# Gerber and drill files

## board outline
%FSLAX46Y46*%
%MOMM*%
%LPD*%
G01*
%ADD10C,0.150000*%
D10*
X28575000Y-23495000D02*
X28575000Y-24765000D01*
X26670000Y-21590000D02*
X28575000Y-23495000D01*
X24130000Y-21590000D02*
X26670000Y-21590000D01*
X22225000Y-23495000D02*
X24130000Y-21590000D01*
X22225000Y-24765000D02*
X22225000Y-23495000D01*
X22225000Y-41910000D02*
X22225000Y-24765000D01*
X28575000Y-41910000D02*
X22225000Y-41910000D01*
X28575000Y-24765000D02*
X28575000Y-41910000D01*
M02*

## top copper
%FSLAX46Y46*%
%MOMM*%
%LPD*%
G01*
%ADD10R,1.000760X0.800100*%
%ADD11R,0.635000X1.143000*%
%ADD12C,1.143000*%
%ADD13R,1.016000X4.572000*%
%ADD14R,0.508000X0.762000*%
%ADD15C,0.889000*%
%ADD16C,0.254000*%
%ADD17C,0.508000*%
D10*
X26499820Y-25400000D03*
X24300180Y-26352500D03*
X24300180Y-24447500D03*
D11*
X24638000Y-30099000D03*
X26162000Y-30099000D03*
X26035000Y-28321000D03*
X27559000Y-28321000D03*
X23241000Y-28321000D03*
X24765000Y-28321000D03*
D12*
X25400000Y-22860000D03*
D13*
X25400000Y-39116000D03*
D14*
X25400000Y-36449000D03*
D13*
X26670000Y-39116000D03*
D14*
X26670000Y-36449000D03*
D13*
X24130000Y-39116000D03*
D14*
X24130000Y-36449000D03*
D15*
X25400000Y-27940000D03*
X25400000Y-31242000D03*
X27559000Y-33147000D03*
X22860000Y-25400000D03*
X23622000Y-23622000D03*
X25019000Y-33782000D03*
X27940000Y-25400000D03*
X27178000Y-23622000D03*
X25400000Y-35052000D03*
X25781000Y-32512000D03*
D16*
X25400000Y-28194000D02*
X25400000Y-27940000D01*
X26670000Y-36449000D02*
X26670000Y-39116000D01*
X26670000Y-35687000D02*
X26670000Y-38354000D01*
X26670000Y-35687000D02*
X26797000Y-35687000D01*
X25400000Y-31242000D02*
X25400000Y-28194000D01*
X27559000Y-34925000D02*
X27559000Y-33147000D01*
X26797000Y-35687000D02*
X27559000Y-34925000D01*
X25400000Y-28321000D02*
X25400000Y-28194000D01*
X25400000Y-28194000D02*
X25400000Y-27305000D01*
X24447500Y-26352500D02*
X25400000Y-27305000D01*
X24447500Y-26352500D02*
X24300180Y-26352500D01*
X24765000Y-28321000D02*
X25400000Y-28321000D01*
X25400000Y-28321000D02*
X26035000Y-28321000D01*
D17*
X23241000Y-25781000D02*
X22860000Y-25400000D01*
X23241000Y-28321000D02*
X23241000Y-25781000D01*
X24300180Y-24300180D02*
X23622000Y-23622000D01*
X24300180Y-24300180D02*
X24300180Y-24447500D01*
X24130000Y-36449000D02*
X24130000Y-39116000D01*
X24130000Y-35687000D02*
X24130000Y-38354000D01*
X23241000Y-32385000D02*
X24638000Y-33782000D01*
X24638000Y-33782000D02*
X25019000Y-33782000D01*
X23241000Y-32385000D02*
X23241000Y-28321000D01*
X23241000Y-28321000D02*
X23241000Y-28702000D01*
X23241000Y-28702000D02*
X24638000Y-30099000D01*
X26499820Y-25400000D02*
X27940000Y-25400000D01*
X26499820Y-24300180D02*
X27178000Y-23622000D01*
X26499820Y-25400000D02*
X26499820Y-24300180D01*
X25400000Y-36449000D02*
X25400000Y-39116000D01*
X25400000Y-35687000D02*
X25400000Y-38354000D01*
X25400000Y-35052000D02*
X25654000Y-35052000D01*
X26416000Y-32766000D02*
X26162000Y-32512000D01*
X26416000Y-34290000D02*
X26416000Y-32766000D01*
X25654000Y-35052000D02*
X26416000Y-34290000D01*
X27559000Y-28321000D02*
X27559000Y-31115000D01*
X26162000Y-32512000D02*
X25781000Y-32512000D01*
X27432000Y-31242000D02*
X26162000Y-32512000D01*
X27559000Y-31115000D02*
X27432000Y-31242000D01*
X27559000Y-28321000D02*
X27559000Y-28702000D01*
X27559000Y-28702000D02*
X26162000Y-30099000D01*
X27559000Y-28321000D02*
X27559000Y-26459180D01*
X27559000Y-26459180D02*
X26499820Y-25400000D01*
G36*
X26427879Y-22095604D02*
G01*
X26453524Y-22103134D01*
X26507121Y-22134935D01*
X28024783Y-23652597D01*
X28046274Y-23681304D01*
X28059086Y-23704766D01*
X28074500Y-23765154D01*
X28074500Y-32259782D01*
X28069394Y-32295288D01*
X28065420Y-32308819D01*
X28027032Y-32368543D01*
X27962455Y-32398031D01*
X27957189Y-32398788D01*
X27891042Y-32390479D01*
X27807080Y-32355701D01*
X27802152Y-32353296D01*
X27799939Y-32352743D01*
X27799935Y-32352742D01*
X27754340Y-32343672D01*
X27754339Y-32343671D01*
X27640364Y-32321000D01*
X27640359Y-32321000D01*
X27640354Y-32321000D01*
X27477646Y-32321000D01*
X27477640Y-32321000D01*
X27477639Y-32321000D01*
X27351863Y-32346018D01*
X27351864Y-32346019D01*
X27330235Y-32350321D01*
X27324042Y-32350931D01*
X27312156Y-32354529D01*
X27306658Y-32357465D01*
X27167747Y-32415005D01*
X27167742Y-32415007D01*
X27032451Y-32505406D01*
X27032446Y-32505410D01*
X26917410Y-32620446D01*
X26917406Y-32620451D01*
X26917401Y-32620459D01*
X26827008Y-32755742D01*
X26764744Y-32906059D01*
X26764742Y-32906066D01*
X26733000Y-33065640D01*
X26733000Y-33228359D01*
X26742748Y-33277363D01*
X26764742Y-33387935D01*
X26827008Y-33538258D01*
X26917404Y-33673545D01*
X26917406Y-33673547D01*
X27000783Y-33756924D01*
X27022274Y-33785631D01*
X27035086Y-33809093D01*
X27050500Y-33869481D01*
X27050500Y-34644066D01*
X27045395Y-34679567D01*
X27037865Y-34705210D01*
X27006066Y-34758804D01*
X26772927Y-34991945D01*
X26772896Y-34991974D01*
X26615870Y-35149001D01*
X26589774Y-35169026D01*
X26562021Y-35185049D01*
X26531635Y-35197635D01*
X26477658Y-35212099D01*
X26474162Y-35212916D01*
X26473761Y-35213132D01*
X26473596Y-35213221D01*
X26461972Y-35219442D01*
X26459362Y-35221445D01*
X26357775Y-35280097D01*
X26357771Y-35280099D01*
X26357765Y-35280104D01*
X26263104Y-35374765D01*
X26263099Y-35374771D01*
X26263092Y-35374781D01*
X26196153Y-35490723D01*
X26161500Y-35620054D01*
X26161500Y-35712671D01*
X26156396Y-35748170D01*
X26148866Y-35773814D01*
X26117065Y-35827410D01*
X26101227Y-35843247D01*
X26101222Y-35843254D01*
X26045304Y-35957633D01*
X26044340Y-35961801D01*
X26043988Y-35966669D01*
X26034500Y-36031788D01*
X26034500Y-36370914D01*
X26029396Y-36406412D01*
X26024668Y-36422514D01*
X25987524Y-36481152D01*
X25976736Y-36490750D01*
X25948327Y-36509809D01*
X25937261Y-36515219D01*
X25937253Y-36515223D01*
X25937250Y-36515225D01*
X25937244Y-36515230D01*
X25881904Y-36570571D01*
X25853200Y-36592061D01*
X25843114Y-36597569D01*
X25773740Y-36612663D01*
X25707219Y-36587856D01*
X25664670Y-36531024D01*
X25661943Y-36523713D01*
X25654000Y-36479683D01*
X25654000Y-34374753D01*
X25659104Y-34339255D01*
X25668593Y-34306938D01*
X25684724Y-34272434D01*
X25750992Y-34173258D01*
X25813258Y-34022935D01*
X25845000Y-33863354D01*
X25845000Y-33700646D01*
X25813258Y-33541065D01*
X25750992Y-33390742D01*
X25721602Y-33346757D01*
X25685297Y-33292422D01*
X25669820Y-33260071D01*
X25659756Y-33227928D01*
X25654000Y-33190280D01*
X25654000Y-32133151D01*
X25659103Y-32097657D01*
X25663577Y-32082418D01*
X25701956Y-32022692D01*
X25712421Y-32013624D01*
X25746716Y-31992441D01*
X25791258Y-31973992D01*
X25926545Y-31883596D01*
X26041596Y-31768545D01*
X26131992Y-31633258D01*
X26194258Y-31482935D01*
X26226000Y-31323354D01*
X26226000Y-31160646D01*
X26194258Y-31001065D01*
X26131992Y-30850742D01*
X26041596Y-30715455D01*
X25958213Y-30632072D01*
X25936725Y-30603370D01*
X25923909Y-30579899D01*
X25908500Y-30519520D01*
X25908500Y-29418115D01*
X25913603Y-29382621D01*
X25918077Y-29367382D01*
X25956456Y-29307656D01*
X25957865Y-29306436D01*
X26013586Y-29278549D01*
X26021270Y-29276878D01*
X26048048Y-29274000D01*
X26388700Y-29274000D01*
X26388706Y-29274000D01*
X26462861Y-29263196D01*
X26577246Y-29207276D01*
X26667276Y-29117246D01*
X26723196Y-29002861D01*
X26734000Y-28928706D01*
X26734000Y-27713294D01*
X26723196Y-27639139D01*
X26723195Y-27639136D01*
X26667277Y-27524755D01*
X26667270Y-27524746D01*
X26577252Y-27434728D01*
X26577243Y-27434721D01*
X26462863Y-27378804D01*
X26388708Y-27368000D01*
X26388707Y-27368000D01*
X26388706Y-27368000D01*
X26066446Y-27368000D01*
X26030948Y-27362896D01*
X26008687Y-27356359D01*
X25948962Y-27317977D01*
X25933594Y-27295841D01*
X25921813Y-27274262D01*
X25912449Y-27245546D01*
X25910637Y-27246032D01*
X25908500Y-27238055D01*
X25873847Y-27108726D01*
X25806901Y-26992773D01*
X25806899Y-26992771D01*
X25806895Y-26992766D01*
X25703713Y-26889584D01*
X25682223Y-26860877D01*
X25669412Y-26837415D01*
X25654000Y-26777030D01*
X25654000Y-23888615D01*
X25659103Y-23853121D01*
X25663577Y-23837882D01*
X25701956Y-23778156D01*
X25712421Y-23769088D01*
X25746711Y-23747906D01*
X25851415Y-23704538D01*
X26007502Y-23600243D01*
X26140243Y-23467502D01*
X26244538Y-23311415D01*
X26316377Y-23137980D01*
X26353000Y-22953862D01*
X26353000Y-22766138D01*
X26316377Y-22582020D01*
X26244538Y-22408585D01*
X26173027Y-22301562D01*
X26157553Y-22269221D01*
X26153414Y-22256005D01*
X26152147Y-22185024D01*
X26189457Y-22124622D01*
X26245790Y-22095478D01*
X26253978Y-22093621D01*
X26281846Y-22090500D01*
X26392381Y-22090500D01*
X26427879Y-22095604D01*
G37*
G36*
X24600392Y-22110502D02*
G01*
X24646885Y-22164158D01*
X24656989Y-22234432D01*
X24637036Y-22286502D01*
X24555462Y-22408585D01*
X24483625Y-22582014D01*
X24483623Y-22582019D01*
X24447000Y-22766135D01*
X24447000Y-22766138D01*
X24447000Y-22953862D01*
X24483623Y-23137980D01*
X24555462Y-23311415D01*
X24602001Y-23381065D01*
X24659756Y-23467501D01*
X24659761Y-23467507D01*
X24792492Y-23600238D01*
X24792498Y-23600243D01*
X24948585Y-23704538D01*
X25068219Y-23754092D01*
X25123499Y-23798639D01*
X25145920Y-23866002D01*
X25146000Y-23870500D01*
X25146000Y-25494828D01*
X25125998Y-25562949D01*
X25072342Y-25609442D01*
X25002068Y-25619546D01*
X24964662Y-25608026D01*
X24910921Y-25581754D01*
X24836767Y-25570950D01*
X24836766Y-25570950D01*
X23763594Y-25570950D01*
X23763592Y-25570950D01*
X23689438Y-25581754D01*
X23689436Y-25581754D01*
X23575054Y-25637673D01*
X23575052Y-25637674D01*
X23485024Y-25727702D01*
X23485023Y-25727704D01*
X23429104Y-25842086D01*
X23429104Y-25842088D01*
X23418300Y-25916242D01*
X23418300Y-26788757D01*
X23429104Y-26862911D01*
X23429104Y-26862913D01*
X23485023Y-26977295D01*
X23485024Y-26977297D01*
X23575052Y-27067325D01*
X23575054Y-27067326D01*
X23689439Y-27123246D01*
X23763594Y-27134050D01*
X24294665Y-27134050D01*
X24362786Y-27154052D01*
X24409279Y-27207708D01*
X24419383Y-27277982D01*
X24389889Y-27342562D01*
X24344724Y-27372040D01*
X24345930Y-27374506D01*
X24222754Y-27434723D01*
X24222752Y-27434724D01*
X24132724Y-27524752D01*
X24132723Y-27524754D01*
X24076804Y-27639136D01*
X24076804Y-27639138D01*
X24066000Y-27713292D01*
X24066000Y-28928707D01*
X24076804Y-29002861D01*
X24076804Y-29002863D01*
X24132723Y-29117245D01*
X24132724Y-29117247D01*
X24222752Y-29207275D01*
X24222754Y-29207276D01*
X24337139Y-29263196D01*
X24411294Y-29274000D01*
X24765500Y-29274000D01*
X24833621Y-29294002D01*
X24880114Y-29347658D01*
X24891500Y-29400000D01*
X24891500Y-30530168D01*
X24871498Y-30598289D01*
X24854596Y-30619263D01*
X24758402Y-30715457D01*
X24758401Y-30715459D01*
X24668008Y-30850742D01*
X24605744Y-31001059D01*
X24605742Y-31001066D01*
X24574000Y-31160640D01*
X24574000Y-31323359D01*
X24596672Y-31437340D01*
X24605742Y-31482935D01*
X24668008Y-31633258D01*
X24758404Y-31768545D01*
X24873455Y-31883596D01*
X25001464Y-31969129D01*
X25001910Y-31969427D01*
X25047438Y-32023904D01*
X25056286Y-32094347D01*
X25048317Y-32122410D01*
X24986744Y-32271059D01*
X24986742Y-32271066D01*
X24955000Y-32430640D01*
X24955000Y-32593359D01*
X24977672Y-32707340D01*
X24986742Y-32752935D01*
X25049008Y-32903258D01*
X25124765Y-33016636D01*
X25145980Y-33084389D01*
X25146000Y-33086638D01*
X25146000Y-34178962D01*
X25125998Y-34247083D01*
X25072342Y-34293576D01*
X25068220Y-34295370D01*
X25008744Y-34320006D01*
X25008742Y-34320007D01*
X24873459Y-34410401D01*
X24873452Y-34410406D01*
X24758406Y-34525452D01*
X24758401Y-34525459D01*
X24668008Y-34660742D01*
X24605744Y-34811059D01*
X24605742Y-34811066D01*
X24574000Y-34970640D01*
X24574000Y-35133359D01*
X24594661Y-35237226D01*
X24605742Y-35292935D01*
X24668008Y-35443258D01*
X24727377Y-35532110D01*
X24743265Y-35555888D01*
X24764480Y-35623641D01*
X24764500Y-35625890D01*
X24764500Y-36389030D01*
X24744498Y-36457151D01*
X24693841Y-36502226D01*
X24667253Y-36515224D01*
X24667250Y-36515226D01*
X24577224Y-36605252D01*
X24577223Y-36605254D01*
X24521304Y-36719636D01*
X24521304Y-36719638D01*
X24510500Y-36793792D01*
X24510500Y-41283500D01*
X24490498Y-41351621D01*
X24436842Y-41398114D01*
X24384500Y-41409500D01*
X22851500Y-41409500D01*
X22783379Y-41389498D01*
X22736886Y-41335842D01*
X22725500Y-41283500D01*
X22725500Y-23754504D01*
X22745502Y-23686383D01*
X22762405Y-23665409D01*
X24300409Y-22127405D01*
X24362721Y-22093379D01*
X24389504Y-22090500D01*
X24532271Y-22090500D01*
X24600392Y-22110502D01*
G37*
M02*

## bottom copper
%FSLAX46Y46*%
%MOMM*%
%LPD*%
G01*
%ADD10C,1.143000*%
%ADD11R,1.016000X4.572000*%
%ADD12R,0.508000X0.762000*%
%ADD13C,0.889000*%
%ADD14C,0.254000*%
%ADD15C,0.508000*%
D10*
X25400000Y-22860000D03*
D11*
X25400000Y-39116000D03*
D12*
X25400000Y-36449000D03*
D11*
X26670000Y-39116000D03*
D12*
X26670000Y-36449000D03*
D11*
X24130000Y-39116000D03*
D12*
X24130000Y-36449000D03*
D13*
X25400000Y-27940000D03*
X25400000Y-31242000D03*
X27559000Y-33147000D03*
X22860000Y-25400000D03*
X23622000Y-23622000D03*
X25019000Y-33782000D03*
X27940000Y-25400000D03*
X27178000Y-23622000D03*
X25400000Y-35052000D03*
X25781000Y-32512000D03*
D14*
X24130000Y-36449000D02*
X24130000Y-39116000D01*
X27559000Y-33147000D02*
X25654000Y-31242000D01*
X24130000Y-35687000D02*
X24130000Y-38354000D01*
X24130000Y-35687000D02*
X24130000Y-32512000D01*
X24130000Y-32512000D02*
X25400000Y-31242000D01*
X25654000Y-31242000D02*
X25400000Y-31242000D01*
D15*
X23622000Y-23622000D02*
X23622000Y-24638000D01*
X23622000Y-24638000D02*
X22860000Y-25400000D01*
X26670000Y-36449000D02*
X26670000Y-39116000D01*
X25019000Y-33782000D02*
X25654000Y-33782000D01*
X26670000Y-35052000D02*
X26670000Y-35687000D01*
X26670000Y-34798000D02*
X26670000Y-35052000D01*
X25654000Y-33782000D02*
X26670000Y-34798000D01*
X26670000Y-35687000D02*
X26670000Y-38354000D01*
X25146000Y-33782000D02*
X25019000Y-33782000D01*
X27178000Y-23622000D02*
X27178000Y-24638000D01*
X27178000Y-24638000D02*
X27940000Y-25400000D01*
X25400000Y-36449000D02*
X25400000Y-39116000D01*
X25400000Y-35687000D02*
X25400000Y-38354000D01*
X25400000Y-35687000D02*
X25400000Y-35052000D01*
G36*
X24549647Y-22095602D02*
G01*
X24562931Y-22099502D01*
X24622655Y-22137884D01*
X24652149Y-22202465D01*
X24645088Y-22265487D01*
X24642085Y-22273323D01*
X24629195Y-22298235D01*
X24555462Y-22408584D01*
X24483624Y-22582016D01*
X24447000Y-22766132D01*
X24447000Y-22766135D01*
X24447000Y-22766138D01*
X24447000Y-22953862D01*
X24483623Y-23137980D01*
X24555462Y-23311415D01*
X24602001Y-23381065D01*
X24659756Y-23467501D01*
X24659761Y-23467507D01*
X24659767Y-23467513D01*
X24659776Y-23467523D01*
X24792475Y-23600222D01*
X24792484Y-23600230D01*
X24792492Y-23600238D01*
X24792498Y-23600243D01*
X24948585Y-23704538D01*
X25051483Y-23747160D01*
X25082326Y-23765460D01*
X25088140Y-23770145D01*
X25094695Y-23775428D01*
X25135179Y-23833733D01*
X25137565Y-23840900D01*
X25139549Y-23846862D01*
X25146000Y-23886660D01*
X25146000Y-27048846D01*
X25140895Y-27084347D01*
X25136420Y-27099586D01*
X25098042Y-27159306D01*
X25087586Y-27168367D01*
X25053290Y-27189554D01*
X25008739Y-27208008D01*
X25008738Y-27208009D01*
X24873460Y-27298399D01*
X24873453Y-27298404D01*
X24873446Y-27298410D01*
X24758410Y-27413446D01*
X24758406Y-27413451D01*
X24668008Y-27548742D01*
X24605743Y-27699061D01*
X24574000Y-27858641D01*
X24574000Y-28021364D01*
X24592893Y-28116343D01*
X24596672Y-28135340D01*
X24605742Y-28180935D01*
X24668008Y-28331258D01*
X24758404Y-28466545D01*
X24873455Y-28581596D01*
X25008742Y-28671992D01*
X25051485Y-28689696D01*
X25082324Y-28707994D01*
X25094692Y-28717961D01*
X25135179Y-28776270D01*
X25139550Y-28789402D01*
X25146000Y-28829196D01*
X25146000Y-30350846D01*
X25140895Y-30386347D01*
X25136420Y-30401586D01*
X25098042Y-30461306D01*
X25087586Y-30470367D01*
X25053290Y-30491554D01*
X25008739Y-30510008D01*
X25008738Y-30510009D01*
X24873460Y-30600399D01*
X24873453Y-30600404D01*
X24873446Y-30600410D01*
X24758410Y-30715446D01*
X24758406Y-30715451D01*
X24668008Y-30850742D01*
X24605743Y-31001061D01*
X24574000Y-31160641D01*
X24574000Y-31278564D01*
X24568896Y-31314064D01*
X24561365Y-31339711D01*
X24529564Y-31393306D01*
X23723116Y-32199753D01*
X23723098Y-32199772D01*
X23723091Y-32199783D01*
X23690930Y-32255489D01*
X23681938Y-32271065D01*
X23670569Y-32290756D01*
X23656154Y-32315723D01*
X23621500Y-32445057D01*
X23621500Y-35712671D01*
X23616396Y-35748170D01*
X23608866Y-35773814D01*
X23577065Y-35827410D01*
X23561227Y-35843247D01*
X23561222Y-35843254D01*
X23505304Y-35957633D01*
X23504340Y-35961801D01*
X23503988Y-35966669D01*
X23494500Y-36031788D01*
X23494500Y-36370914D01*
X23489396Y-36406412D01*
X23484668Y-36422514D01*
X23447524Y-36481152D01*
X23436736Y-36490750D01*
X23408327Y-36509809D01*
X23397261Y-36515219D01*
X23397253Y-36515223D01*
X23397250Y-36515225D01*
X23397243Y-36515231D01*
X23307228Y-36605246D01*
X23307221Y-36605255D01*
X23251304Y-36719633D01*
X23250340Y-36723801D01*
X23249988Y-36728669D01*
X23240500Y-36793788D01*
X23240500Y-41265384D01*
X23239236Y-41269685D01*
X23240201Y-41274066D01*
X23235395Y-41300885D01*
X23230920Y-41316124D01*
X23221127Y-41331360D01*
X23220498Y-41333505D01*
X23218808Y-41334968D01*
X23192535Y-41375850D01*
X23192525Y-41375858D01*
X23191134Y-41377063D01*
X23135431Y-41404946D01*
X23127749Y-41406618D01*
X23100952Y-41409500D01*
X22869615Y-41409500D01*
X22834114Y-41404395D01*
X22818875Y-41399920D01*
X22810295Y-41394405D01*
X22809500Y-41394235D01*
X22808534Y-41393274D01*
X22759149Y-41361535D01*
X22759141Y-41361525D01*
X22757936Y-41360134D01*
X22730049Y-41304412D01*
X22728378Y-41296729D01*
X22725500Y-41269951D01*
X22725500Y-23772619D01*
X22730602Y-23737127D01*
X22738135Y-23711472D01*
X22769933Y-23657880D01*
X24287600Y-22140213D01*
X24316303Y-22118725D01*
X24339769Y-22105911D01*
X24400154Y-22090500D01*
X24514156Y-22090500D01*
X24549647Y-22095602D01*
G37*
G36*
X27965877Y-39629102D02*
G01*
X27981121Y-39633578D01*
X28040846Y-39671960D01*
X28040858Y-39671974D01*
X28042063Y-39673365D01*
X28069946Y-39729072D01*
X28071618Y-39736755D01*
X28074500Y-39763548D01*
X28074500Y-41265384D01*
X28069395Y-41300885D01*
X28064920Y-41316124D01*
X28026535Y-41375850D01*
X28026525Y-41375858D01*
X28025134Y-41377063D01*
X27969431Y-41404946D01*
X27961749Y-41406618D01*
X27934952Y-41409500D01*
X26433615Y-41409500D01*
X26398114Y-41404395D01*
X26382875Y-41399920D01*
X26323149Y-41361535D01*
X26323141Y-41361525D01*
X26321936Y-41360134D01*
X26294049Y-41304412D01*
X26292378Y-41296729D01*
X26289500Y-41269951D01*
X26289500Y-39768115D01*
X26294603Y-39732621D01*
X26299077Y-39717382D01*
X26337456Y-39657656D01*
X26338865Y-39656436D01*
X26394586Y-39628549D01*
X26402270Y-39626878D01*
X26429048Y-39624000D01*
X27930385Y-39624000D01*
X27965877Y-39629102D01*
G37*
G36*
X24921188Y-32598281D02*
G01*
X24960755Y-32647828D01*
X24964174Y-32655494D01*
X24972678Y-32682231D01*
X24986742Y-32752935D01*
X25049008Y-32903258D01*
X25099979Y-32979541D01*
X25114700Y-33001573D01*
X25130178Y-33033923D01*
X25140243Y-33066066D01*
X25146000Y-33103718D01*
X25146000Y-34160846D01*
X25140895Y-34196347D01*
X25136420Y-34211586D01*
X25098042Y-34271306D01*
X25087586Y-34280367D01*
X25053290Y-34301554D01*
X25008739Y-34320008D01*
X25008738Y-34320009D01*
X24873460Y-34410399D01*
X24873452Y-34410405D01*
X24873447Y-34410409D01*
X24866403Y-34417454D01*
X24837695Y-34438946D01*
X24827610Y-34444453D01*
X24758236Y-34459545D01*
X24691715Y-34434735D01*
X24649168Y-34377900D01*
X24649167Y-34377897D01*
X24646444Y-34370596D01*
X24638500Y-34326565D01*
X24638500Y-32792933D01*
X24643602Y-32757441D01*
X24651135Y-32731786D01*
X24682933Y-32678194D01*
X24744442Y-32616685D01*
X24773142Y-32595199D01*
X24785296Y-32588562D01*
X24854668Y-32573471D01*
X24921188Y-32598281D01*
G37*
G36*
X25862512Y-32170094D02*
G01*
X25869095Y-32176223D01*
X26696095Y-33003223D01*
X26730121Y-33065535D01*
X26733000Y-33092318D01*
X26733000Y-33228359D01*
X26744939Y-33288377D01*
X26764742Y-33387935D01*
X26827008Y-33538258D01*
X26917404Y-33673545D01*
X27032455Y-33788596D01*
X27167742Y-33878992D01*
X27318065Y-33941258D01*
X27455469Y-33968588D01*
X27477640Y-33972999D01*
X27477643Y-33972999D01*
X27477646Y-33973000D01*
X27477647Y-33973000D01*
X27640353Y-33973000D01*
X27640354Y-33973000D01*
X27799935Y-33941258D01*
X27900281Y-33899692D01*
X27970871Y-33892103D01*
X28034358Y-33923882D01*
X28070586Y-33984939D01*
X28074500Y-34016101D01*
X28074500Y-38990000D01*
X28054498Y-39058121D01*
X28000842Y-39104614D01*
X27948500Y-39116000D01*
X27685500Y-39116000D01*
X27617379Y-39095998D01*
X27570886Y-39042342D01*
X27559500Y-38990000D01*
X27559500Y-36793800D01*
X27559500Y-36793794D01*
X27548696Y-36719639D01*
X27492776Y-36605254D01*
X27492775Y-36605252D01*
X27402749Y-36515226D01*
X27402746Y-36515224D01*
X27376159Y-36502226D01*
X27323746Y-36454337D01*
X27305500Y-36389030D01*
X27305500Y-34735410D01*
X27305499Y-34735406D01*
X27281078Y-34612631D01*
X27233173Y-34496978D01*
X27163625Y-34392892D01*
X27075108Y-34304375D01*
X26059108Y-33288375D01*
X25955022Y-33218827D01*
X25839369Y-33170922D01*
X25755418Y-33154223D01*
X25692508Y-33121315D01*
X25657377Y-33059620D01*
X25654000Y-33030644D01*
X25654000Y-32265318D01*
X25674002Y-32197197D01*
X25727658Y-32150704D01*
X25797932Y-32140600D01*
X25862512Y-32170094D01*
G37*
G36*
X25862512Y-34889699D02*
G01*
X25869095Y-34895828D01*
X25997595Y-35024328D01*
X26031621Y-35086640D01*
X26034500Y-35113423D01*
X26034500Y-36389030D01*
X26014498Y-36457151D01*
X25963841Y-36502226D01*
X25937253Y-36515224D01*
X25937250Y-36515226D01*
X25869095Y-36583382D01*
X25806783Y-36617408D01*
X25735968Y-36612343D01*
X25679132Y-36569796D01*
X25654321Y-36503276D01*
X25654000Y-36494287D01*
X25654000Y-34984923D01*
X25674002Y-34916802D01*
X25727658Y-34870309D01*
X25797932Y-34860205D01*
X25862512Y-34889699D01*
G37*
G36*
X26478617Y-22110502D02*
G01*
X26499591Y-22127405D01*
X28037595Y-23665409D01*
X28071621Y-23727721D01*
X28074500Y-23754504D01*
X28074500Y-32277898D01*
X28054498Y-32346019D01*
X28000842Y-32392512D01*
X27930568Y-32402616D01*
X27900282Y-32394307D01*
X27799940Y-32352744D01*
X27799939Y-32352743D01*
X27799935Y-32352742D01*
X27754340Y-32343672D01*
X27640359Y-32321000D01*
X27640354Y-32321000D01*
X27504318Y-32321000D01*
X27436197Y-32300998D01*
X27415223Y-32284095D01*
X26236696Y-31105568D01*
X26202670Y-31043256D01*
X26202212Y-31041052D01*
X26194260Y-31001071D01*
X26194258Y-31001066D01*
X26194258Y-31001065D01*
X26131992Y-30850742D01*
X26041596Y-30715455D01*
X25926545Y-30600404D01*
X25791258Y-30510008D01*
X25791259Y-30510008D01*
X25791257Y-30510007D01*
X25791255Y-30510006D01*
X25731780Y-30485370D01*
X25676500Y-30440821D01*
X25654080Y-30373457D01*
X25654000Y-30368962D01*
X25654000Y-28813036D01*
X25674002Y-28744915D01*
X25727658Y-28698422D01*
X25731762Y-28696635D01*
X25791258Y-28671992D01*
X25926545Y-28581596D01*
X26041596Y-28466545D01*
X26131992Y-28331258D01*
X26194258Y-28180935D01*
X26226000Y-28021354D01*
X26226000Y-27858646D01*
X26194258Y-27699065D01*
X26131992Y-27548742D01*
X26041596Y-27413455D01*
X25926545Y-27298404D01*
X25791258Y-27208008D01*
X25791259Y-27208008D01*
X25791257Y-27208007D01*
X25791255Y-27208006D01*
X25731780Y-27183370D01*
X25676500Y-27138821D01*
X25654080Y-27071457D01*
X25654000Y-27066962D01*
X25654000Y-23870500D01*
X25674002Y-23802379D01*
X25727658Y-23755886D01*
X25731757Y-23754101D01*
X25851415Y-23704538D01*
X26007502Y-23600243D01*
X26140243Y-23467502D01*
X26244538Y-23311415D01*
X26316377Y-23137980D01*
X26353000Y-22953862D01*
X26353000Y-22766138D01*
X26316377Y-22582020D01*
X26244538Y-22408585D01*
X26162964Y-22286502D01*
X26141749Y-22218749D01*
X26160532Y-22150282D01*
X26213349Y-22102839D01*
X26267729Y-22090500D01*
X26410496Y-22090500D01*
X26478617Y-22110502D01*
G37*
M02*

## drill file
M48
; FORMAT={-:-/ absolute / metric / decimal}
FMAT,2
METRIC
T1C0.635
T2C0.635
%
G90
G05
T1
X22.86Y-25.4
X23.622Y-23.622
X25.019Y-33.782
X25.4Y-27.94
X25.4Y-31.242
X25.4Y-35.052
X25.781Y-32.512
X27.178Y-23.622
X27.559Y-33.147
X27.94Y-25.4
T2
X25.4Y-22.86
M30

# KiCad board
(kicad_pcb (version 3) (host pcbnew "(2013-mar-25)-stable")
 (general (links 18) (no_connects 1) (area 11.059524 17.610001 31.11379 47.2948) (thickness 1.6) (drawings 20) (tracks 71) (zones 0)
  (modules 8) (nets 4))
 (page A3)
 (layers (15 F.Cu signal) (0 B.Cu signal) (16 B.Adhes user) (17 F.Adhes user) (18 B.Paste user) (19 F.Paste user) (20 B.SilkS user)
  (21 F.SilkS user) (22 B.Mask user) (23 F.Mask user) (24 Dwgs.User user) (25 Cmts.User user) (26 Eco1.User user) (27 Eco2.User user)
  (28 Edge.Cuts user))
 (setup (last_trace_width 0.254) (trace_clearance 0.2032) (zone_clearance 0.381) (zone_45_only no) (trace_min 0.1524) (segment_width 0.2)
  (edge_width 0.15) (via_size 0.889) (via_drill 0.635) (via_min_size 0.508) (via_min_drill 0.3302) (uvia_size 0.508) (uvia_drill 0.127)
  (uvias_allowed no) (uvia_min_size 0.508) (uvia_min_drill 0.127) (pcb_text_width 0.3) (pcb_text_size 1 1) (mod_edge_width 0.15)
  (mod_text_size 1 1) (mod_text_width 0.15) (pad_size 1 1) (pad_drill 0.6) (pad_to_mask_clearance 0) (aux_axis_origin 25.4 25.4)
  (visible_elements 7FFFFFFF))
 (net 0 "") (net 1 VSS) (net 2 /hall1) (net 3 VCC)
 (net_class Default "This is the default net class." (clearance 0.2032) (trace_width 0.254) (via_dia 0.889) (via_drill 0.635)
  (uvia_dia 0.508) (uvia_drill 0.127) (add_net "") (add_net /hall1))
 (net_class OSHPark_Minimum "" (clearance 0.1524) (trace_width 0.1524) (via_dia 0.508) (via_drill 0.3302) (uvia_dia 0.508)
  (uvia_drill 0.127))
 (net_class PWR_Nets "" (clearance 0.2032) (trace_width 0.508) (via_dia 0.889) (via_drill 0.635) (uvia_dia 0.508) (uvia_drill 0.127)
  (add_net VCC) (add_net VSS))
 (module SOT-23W (layer F.Cu) (at 25.4 25.4 270)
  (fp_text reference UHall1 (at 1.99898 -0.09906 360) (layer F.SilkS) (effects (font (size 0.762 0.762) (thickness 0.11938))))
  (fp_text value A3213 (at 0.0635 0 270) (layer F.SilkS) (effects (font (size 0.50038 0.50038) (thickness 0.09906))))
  (pad 2 smd rect (at 0 -1.09982 270) (size 0.8001 1.00076) (layers F.Cu F.Paste F.Mask) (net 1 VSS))
  (pad 3 smd rect (at 0.9525 1.09982 270) (size 0.8001 1.00076) (layers F.Cu F.Paste F.Mask) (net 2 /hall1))
  (pad 1 smd rect (at -0.9525 1.09982 270) (size 0.8001 1.00076) (layers F.Cu F.Paste F.Mask) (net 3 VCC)))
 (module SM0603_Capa (layer F.Cu) (at 25.4 30.099)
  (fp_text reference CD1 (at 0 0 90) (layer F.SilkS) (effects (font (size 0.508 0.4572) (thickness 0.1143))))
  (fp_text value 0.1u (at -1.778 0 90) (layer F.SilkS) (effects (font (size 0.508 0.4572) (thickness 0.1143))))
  (pad 1 smd rect (at -0.762 0) (size 0.635 1.143) (layers F.Cu F.Paste F.Mask) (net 3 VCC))
  (pad 2 smd rect (at 0.762 0) (size 0.635 1.143) (layers F.Cu F.Paste F.Mask) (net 1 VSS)))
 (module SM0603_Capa (layer F.Cu) (at 26.797 28.321)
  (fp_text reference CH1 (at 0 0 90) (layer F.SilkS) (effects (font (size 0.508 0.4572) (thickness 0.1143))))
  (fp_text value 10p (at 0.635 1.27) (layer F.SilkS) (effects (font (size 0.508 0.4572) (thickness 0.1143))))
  (pad 1 smd rect (at -0.762 0) (size 0.635 1.143) (layers F.Cu F.Paste F.Mask) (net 2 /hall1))
  (pad 2 smd rect (at 0.762 0) (size 0.635 1.143) (layers F.Cu F.Paste F.Mask) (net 1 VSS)))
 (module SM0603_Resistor (layer F.Cu) (at 24.003 28.321)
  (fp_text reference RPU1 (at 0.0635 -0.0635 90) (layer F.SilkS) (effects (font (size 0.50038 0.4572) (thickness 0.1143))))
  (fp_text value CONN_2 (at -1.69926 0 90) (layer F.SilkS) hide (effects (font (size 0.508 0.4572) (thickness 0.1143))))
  (pad 1 smd rect (at -0.762 0) (size 0.635 1.143) (layers F.Cu F.Paste F.Mask) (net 3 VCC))
  (pad 2 smd rect (at 0.762 0) (size 0.635 1.143) (layers F.Cu F.Paste F.Mask) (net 2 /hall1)))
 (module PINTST (layer F.Cu) (at 25.4 22.86)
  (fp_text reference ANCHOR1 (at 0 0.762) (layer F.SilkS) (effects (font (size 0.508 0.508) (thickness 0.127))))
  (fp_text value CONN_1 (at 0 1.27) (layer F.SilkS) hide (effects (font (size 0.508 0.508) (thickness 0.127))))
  (pad 1 thru_hole circle (at 0 0) (size 1.143 1.143) (drill 0.635) (layers *.Cu *.Mask F.SilkS)))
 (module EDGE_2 (layer F.Cu) (at 25.4 38.862 180)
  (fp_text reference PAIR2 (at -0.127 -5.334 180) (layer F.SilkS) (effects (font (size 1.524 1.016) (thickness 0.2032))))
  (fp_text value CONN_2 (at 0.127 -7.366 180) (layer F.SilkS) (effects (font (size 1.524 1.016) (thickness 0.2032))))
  (pad 1 connect rect (at 0 -0.254 180) (size 1.016 4.572) (layers F.Cu F.Mask) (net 1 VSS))
  (pad 2 connect rect (at 0 -0.254 180) (size 1.016 4.572) (layers B.Cu B.Mask) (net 1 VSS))
  (pad 1 connect rect (at 0 2.413 180) (size 0.508 0.762) (layers F.Cu F.Mask) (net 1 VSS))
  (pad 2 connect rect (at 0 2.413 180) (size 0.508 0.762) (layers B.Cu B.Mask) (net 1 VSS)))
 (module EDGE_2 (layer F.Cu) (at 26.67 38.862 180)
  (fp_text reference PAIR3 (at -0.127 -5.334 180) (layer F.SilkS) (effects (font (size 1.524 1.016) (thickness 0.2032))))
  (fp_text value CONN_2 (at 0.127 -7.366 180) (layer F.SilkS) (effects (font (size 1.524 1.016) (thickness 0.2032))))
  (pad 1 connect rect (at 0 -0.254 180) (size 1.016 4.572) (layers F.Cu F.Mask) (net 2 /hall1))
  (pad 2 connect rect (at 0 -0.254 180) (size 1.016 4.572) (layers B.Cu B.Mask) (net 3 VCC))
  (pad 1 connect rect (at 0 2.413 180) (size 0.508 0.762) (layers F.Cu F.Mask) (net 2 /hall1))
  (pad 2 connect rect (at 0 2.413 180) (size 0.508 0.762) (layers B.Cu B.Mask) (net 3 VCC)))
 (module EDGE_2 (layer F.Cu) (at 24.13 38.862 180)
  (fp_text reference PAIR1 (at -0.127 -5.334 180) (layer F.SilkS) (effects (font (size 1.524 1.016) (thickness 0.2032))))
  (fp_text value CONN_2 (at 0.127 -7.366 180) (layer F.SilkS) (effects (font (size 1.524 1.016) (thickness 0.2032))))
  (pad 1 connect rect (at 0 -0.254 180) (size 1.016 4.572) (layers F.Cu F.Mask) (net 3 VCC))
  (pad 2 connect rect (at 0 -0.254 180) (size 1.016 4.572) (layers B.Cu B.Mask) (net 2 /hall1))
  (pad 1 connect rect (at 0 2.413 180) (size 0.508 0.762) (layers F.Cu F.Mask) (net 3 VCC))
  (pad 2 connect rect (at 0 2.413 180) (size 0.508 0.762) (layers B.Cu B.Mask) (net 2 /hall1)))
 (gr_line (start 28.575 23.495) (end 28.575 24.765) (angle 90) (layer Edge.Cuts) (width 0.15))
 (gr_line (start 26.67 21.59) (end 28.575 23.495) (angle 90) (layer Edge.Cuts) (width 0.15))
 (gr_line (start 24.13 21.59) (end 26.67 21.59) (angle 90) (layer Edge.Cuts) (width 0.15))
 (gr_line (start 22.225 23.495) (end 24.13 21.59) (angle 90) (layer Edge.Cuts) (width 0.15))
 (gr_line (start 22.225 24.765) (end 22.225 23.495) (angle 90) (layer Edge.Cuts) (width 0.15))
 (gr_line (start 22.225 41.91) (end 22.225 24.765) (angle 90) (layer Edge.Cuts) (width 0.15))
 (gr_line (start 28.575 41.91) (end 22.225 41.91) (angle 90) (layer Edge.Cuts) (width 0.15))
 (gr_line (start 28.575 24.765) (end 28.575 41.91) (angle 90) (layer Edge.Cuts) (width 0.15))
 (segment (start 25.4 28.194) (end 25.4 27.94) (width 0.254) (layer F.Cu) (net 2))
 (via (at 25.4 27.94) (size 0.889) (layers F.Cu B.Cu) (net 2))
 (segment (start 26.67 36.449) (end 26.67 39.116) (width 0.254) (layer F.Cu) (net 2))
 (segment (start 24.13 36.449) (end 24.13 39.116) (width 0.254) (layer B.Cu) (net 2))
 (segment (start 27.559 33.147) (end 25.654 31.242) (width 0.254) (layer B.Cu) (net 2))
 (segment (start 26.67 35.687) (end 26.67 38.354) (width 0.254) (layer F.Cu) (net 2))
 (segment (start 24.13 35.687) (end 24.13 38.354) (width 0.254) (layer B.Cu) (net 2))
 (segment (start 24.13 35.687) (end 24.13 32.512) (width 0.254) (layer B.Cu) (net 2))
 (segment (start 24.13 32.512) (end 25.4 31.242) (width 0.254) (layer B.Cu) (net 2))
 (segment (start 26.67 35.687) (end 26.797 35.687) (width 0.254) (layer F.Cu) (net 2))
 (segment (start 25.4 31.242) (end 25.4 28.194) (width 0.254) (layer F.Cu) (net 2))
 (via (at 25.4 31.242) (size 0.889) (layers F.Cu B.Cu) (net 2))
 (segment (start 25.654 31.242) (end 25.4 31.242) (width 0.254) (layer B.Cu) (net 2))
 (via (at 27.559 33.147) (size 0.889) (layers F.Cu B.Cu) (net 2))
 (segment (start 27.559 34.925) (end 27.559 33.147) (width 0.254) (layer F.Cu) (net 2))
 (segment (start 26.797 35.687) (end 27.559 34.925) (width 0.254) (layer F.Cu) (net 2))
 (segment (start 25.4 28.321) (end 25.4 28.194) (width 0.254) (layer F.Cu) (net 2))
 (segment (start 25.4 28.194) (end 25.4 27.305) (width 0.254) (layer F.Cu) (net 2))
 (segment (start 24.4475 26.3525) (end 25.4 27.305) (width 0.254) (layer F.Cu) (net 2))
 (segment (start 24.4475 26.3525) (end 24.30018 26.3525) (width 0.254) (layer F.Cu) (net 2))
 (segment (start 24.765 28.321) (end 25.4 28.321) (width 0.254) (layer F.Cu) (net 2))
 (segment (start 25.4 28.321) (end 26.035 28.321) (width 0.254) (layer F.Cu) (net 2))
 (segment (start 23.622 23.622) (end 23.622 24.638) (width 0.508) (layer B.Cu) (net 3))
 (via (at 22.86 25.4) (size 0.889) (layers F.Cu B.Cu) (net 3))
 (segment (start 23.241 25.781) (end 22.86 25.4) (width 0.508) (layer F.Cu) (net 3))
 (segment (start 23.241 28.321) (end 23.241 25.781) (width 0.508) (layer F.Cu) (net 3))
 (segment (start 24.30018 24.30018) (end 23.622 23.622) (width 0.508) (layer F.Cu) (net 3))
 (via (at 23.622 23.622) (size 0.889) (layers F.Cu B.Cu) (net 3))
 (segment (start 24.30018 24.30018) (end 24.30018 24.4475) (width 0.508) (layer F.Cu) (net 3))
 (segment (start 23.622 24.638) (end 22.86 25.4) (width 0.508) (layer B.Cu) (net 3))
 (segment (start 24.13 36.449) (end 24.13 39.116) (width 0.508) (layer F.Cu) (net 3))
 (segment (start 26.67 36.449) (end 26.67 39.116) (width 0.508) (layer B.Cu) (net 3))
 (segment (start 24.13 35.687) (end 24.13 38.354) (width 0.508) (layer F.Cu) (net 3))
 (segment (start 25.019 33.782) (end 25.654 33.782) (width 0.508) (layer B.Cu) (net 3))
 (segment (start 26.67 35.052) (end 26.67 35.687) (width 0.508) (layer B.Cu) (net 3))
 (segment (start 26.67 34.798) (end 26.67 35.052) (width 0.508) (layer B.Cu) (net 3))
 (segment (start 25.654 33.782) (end 26.67 34.798) (width 0.508) (layer B.Cu) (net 3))
 (segment (start 26.67 35.687) (end 26.67 38.354) (width 0.508) (layer B.Cu) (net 3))
 (segment (start 23.241 32.385) (end 24.638 33.782) (width 0.508) (layer F.Cu) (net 3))
 (segment (start 24.638 33.782) (end 25.019 33.782) (width 0.508) (layer F.Cu) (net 3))
 (via (at 25.019 33.782) (size 0.889) (layers F.Cu B.Cu) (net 3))
 (segment (start 23.241 32.385) (end 23.241 28.321) (width 0.508) (layer F.Cu) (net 3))
 (segment (start 25.146 33.782) (end 25.019 33.782) (width 0.508) (layer B.Cu) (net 3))
 (segment (start 23.241 28.321) (end 23.241 28.702) (width 0.508) (layer F.Cu) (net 3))
 (segment (start 23.241 28.702) (end 24.638 30.099) (width 0.508) (layer F.Cu) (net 3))
 (segment (start 27.178 23.622) (end 27.178 24.638) (width 0.508) (layer B.Cu) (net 1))
 (via (at 27.94 25.4) (size 0.889) (layers F.Cu B.Cu) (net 1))
 (segment (start 26.49982 25.4) (end 27.94 25.4) (width 0.508) (layer F.Cu) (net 1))
 (segment (start 26.49982 24.30018) (end 27.178 23.622) (width 0.508) (layer F.Cu) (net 1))
 (via (at 27.178 23.622) (size 0.889) (layers F.Cu B.Cu) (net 1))
 (segment (start 26.49982 25.4) (end 26.49982 24.30018) (width 0.508) (layer F.Cu) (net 1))
 (segment (start 27.178 24.638) (end 27.94 25.4) (width 0.508) (layer B.Cu) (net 1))
 (segment (start 25.4 36.449) (end 25.4 39.116) (width 0.508) (layer F.Cu) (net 1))
 (segment (start 25.4 36.449) (end 25.4 39.116) (width 0.508) (layer B.Cu) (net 1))
 (segment (start 25.4 35.687) (end 25.4 38.354) (width 0.508) (layer F.Cu) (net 1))
 (segment (start 25.4 35.687) (end 25.4 38.354) (width 0.508) (layer B.Cu) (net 1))
 (segment (start 25.4 35.052) (end 25.654 35.052) (width 0.508) (layer F.Cu) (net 1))
 (via (at 25.4 35.052) (size 0.889) (layers F.Cu B.Cu) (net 1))
 (segment (start 25.4 35.687) (end 25.4 35.052) (width 0.508) (layer B.Cu) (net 1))
 (segment (start 26.416 32.766) (end 26.162 32.512) (width 0.508) (layer F.Cu) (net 1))
 (segment (start 26.416 34.29) (end 26.416 32.766) (width 0.508) (layer F.Cu) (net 1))
 (segment (start 25.654 35.052) (end 26.416 34.29) (width 0.508) (layer F.Cu) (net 1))
 (segment (start 27.559 28.321) (end 27.559 31.115) (width 0.508) (layer F.Cu) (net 1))
 (via (at 25.781 32.512) (size 0.889) (layers F.Cu B.Cu) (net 1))
 (segment (start 26.162 32.512) (end 25.781 32.512) (width 0.508) (layer F.Cu) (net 1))
 (segment (start 27.432 31.242) (end 26.162 32.512) (width 0.508) (layer F.Cu) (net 1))
 (segment (start 27.559 31.115) (end 27.432 31.242) (width 0.508) (layer F.Cu) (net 1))
 (segment (start 27.559 28.321) (end 27.559 28.702) (width 0.508) (layer F.Cu) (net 1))
 (segment (start 27.559 28.702) (end 26.162 30.099) (width 0.508) (layer F.Cu) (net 1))
 (segment (start 27.559 28.321) (end 27.559 26.45918) (width 0.508) (layer F.Cu) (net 1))
 (segment (start 27.559 26.45918) (end 26.49982 25.4) (width 0.508) (layer F.Cu) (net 1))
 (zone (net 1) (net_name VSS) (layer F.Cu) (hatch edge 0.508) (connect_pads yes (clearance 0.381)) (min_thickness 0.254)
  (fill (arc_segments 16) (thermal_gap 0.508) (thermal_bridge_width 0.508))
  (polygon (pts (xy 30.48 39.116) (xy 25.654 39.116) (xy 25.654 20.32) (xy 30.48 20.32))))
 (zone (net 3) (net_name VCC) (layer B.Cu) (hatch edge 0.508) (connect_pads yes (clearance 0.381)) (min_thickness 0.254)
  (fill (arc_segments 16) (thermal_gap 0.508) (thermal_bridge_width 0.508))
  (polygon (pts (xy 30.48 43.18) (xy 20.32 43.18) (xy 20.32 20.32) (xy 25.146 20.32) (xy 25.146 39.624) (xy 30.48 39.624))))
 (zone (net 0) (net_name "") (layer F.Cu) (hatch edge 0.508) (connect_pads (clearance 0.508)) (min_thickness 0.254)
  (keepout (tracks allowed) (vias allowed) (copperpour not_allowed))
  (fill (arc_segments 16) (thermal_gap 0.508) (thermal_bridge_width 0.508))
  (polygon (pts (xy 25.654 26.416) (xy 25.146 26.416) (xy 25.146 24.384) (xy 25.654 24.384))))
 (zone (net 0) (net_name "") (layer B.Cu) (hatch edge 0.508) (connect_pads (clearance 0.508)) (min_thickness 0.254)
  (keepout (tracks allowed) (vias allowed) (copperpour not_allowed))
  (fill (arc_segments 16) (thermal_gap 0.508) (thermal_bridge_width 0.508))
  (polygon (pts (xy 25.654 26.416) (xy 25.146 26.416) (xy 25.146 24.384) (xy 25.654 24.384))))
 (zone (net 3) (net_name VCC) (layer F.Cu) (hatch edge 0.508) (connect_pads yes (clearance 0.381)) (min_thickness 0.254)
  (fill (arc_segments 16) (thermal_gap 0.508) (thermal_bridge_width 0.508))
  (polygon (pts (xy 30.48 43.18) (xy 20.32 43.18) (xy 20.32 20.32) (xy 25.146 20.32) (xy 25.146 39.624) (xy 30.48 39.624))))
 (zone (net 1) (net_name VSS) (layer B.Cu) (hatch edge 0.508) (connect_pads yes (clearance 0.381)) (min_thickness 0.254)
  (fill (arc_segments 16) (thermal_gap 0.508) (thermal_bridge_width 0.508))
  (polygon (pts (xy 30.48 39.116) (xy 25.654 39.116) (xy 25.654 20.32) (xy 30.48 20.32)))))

